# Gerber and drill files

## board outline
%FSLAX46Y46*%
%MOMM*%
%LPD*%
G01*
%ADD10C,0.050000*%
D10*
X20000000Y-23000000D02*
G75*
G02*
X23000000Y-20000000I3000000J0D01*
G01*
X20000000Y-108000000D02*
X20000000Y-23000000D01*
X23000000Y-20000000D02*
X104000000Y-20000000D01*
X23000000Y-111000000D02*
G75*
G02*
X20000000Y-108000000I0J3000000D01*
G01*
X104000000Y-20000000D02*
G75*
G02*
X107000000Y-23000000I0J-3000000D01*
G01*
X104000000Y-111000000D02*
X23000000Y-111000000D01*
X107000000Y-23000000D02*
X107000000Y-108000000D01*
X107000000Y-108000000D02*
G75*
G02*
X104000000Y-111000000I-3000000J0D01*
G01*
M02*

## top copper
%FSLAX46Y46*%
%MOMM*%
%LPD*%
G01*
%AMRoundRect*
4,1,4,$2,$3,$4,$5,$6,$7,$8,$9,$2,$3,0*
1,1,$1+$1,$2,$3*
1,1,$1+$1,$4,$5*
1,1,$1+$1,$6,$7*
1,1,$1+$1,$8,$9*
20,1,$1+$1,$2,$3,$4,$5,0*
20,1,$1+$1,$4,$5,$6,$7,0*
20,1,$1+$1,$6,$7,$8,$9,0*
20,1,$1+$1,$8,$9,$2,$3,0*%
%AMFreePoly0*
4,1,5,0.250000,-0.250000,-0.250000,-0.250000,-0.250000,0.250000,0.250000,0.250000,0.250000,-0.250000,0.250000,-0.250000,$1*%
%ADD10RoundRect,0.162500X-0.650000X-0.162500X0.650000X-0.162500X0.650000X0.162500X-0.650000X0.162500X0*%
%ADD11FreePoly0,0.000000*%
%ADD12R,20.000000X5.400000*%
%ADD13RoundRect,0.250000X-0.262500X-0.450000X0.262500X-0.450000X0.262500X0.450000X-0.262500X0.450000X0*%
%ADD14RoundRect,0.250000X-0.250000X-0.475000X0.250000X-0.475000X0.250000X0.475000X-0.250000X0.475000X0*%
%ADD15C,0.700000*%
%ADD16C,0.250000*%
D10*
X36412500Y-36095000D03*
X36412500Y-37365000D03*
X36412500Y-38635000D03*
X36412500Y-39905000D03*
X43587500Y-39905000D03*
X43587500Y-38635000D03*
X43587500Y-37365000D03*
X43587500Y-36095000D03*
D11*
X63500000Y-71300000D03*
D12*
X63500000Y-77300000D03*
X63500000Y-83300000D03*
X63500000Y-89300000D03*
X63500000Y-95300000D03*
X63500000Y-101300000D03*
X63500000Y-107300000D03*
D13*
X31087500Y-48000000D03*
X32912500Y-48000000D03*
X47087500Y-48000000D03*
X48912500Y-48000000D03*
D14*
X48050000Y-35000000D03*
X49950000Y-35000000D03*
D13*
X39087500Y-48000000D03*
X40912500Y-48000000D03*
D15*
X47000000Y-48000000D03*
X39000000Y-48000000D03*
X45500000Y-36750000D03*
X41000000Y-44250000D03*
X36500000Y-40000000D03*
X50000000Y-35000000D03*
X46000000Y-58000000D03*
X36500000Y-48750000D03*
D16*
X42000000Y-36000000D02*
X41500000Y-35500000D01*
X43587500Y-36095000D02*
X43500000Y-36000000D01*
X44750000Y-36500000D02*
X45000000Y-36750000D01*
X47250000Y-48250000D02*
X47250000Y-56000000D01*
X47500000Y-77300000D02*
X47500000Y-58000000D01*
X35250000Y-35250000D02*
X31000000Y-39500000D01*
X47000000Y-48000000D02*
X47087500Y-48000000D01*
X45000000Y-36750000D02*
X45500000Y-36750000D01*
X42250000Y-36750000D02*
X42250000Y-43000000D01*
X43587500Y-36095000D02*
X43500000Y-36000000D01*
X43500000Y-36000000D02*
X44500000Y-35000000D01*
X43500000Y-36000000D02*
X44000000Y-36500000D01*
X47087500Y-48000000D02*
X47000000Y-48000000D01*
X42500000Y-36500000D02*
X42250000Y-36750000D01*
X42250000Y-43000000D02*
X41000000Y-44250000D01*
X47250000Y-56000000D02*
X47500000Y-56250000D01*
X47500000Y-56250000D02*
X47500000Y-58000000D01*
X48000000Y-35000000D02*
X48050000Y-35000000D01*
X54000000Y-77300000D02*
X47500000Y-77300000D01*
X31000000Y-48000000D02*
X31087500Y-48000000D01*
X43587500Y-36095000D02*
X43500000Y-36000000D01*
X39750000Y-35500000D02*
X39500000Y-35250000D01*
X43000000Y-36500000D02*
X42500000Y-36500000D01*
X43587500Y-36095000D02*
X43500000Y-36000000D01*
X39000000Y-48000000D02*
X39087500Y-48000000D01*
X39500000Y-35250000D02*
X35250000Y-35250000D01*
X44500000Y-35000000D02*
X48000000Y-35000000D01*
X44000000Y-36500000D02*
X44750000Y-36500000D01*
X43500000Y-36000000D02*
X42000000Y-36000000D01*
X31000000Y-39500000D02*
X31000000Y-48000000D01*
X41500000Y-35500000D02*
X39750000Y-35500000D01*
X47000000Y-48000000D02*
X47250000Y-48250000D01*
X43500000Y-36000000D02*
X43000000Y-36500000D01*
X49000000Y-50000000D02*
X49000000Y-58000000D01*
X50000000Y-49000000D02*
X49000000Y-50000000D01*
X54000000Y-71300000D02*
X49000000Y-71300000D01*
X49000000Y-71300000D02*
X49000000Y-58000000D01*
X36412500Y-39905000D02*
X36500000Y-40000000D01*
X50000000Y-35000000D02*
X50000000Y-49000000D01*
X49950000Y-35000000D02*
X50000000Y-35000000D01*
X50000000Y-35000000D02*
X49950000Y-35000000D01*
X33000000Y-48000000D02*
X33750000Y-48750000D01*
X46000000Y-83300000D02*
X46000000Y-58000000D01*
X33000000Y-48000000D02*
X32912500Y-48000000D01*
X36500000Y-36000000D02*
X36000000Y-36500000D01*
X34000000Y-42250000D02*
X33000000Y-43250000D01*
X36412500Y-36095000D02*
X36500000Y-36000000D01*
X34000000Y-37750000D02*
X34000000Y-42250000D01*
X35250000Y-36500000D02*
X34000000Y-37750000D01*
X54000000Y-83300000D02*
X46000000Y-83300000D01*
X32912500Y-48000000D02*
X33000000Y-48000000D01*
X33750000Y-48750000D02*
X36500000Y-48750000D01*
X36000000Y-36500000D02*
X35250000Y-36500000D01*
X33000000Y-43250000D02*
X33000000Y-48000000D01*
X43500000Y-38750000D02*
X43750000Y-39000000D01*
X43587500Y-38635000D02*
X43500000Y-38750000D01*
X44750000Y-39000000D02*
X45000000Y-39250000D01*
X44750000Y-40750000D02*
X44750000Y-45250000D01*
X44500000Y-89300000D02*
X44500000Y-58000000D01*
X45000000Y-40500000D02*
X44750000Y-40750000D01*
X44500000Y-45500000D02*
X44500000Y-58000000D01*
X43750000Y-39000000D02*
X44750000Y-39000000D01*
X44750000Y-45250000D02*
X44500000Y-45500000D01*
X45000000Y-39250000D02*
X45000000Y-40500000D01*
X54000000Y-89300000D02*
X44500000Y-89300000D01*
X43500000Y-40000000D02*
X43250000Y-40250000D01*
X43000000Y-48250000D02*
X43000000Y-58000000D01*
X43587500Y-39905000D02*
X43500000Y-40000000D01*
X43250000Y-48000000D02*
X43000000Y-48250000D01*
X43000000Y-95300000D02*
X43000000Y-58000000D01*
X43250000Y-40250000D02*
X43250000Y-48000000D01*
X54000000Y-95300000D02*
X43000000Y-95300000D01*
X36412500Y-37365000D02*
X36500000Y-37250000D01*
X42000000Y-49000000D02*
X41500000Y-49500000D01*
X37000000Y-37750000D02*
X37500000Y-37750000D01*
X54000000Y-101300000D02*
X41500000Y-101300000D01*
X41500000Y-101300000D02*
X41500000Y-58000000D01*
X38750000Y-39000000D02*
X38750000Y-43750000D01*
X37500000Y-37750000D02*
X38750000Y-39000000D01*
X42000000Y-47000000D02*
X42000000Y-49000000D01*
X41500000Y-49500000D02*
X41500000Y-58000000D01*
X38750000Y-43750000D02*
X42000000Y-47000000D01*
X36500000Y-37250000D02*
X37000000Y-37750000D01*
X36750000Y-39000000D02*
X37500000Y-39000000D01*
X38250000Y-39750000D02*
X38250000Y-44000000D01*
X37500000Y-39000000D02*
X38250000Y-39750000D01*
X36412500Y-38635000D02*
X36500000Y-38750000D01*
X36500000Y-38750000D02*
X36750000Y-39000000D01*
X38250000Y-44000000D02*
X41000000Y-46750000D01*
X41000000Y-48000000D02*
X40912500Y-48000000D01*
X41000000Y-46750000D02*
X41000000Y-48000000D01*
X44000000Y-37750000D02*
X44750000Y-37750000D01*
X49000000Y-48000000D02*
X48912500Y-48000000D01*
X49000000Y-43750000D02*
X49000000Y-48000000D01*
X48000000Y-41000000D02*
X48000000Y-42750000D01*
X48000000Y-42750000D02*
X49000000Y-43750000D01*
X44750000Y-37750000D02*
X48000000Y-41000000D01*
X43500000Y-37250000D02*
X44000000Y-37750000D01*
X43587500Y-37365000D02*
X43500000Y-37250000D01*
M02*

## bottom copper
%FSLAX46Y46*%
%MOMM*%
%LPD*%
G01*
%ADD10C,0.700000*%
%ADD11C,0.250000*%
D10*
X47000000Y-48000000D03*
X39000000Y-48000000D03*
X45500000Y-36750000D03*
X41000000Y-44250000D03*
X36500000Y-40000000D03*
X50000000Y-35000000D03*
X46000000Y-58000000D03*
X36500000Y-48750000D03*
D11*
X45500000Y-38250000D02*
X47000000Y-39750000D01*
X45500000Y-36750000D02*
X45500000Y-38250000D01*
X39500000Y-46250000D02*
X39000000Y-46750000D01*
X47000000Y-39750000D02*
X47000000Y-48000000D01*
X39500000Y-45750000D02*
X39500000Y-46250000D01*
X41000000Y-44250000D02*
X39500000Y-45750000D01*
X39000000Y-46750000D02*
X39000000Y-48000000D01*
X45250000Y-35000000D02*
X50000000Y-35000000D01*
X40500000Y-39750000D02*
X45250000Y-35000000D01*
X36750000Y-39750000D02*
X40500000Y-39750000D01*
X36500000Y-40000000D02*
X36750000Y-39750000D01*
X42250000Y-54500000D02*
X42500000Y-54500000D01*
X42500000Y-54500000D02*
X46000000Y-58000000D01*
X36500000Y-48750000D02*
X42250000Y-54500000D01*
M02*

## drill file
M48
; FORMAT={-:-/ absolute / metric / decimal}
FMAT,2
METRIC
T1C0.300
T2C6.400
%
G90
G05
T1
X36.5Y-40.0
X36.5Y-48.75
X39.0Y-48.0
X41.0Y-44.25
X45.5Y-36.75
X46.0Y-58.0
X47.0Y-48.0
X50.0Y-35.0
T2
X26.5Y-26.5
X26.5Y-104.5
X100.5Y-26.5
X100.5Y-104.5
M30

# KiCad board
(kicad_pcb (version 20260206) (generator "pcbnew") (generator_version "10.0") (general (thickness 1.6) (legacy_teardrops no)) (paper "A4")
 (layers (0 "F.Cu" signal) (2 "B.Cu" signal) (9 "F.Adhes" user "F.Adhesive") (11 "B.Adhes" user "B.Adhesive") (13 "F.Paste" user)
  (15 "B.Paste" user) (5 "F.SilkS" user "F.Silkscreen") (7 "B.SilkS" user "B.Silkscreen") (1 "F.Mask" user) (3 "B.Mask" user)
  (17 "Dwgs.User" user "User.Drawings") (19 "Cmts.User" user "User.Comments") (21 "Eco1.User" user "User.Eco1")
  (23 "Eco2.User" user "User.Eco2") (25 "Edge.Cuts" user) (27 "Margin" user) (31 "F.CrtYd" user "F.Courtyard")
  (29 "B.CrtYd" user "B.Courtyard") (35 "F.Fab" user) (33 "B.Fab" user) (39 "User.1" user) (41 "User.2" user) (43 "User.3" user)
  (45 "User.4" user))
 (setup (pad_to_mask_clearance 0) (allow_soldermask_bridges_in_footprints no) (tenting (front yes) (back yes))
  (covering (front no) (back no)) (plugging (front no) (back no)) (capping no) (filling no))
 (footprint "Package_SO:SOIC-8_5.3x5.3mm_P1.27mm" (layer "F.Cu") (at 40 38)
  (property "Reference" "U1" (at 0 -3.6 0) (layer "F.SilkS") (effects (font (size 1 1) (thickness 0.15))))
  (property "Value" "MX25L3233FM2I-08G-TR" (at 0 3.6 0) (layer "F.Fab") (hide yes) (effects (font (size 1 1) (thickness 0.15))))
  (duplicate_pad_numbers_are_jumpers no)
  (pad "1" smd roundrect (at -3.5875 -1.905) (size 1.625 0.65) (layers "F.Cu" "F.Mask" "F.Paste") (roundrect_rratio 0.25) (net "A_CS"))
  (pad "2" smd roundrect (at -3.5875 -0.635) (size 1.625 0.65) (layers "F.Cu" "F.Mask" "F.Paste") (roundrect_rratio 0.25) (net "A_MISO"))
  (pad "3" smd roundrect (at -3.5875 0.635) (size 1.625 0.65) (layers "F.Cu" "F.Mask" "F.Paste") (roundrect_rratio 0.25) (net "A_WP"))
  (pad "4" smd roundrect (at -3.5875 1.905) (size 1.625 0.65) (layers "F.Cu" "F.Mask" "F.Paste") (roundrect_rratio 0.25) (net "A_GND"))
  (pad "5" smd roundrect (at 3.5875 1.905) (size 1.625 0.65) (layers "F.Cu" "F.Mask" "F.Paste") (roundrect_rratio 0.25) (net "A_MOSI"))
  (pad "6" smd roundrect (at 3.5875 0.635) (size 1.625 0.65) (layers "F.Cu" "F.Mask" "F.Paste") (roundrect_rratio 0.25) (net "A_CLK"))
  (pad "7" smd roundrect (at 3.5875 -0.635) (size 1.625 0.65) (layers "F.Cu" "F.Mask" "F.Paste") (roundrect_rratio 0.25) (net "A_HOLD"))
  (pad "8" smd roundrect (at 3.5875 -1.905) (size 1.625 0.65) (layers "F.Cu" "F.Mask" "F.Paste") (roundrect_rratio 0.25) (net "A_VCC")))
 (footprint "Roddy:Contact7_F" (layer "F.Cu") (at 63.5 0)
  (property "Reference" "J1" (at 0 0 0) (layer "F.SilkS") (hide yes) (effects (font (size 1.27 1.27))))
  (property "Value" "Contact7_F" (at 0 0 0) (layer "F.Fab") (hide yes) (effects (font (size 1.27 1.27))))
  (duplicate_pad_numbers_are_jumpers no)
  (pad "1" smd custom (at 0 71.3) (size 0.5 0.5) (layers "F.Cu" "F.Mask") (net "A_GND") (solder_mask_margin 0.05) (thermal_bridge_angle 45)
   (options (clearance outline) (anchor rect)) (primitives))
  (pad "2" smd rect (at 0 77.3) (size 20 5.4) (layers "F.Cu" "F.Mask") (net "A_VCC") (solder_mask_margin 0.05) (thermal_bridge_angle 45))
  (pad "3" smd rect (at 0 83.3) (size 20 5.4) (layers "F.Cu" "F.Mask") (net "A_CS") (solder_mask_margin 0.05) (thermal_bridge_angle 45))
  (pad "4" smd rect (at 0 89.3) (size 20 5.4) (layers "F.Cu" "F.Mask") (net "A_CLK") (solder_mask_margin 0.05) (thermal_bridge_angle 45))
  (pad "5" smd rect (at 0 95.3) (size 20 5.4) (layers "F.Cu" "F.Mask") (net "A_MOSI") (solder_mask_margin 0.05) (thermal_bridge_angle 45))
  (pad "6" smd rect (at 0 101.3) (size 20 5.4) (layers "F.Cu" "F.Mask") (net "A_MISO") (solder_mask_margin 0.05) (thermal_bridge_angle 45))
  (pad "7" smd rect (at 0 107.3) (size 20 5.4) (layers "F.Cu" "F.Mask") (solder_mask_margin 0.05) (thermal_bridge_angle 45)))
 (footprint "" (layer "F.Cu") (at 100.5 26.5)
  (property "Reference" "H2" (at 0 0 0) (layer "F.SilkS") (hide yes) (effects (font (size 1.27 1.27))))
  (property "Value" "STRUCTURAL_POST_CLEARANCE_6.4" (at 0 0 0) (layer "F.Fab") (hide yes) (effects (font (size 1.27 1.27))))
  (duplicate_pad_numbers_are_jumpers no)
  (pad "" np_thru_hole circle (at 0 0) (size 6.4 6.4) (drill 6.4) (layers "*.Cu")))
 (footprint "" (layer "F.Cu") (at 26.5 26.5)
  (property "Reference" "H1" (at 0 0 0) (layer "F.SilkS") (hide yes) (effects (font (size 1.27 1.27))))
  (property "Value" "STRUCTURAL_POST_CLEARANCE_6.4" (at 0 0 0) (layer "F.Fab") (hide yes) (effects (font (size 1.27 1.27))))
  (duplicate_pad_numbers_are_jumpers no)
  (pad "" np_thru_hole circle (at 0 0) (size 6.4 6.4) (drill 6.4) (layers "*.Cu")))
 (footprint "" (layer "F.Cu") (at 26.5 104.5)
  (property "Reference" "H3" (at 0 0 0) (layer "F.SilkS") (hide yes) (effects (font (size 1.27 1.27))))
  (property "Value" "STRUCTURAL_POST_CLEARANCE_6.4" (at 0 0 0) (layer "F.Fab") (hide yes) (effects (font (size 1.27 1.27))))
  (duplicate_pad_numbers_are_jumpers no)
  (pad "" np_thru_hole circle (at 0 0) (size 6.4 6.4) (drill 6.4) (layers "*.Cu")))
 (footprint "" (layer "F.Cu") (at 100.5 104.5)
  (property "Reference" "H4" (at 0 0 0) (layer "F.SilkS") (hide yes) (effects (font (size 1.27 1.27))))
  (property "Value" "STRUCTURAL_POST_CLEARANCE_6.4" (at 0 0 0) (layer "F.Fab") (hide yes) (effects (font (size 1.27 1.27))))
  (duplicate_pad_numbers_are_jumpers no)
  (pad "" np_thru_hole circle (at 0 0) (size 6.4 6.4) (drill 6.4) (layers "*.Cu")))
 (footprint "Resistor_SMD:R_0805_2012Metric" (layer "F.Cu") (at 32 48)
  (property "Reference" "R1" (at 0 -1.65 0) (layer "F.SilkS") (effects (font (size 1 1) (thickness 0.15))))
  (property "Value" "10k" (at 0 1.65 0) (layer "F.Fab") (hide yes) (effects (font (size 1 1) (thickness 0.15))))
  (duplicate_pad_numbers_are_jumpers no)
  (pad "1" smd roundrect (at -0.9125 0) (size 1.025 1.4) (layers "F.Cu" "F.Mask" "F.Paste") (roundrect_rratio 0.243902) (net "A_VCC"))
  (pad "2" smd roundrect (at 0.9125 0) (size 1.025 1.4) (layers "F.Cu" "F.Mask" "F.Paste") (roundrect_rratio 0.243902) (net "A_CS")))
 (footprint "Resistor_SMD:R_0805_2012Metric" (layer "F.Cu") (at 48 48)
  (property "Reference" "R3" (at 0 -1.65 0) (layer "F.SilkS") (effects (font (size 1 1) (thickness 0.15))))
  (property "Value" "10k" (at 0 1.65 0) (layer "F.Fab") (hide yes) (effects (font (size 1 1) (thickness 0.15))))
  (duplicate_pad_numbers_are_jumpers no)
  (pad "1" smd roundrect (at -0.9125 0) (size 1.025 1.4) (layers "F.Cu" "F.Mask" "F.Paste") (roundrect_rratio 0.243902) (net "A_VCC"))
  (pad "2" smd roundrect (at 0.9125 0) (size 1.025 1.4) (layers "F.Cu" "F.Mask" "F.Paste") (roundrect_rratio 0.243902) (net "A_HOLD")))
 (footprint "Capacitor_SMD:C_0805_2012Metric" (layer "F.Cu") (at 49 35)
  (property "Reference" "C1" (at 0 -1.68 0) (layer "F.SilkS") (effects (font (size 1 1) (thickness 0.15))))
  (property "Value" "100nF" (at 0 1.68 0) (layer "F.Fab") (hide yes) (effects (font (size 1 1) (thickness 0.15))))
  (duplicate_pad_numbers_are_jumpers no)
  (pad "1" smd roundrect (at -0.95 0) (size 1 1.45) (layers "F.Cu" "F.Mask" "F.Paste") (roundrect_rratio 0.25) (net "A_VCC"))
  (pad "2" smd roundrect (at 0.95 0) (size 1 1.45) (layers "F.Cu" "F.Mask" "F.Paste") (roundrect_rratio 0.25) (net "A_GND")))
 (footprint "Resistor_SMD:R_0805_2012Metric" (layer "F.Cu") (at 40 48)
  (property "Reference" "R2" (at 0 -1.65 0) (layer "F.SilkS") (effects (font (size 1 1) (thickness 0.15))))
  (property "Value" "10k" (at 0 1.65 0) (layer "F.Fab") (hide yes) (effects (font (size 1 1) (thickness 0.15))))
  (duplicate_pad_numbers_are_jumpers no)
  (pad "1" smd roundrect (at -0.9125 0) (size 1.025 1.4) (layers "F.Cu" "F.Mask" "F.Paste") (roundrect_rratio 0.243902) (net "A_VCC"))
  (pad "2" smd roundrect (at 0.9125 0) (size 1.025 1.4) (layers "F.Cu" "F.Mask" "F.Paste") (roundrect_rratio 0.243902) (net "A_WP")))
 (gr_arc (start 20 23) (mid 20.878679 20.878679) (end 23 20) (stroke (width 0.05) (type default)) (layer "Edge.Cuts"))
 (gr_line (start 20 108) (end 20 23) (stroke (width 0.05) (type default)) (layer "Edge.Cuts"))
 (gr_line (start 23 20) (end 104 20) (stroke (width 0.05) (type default)) (layer "Edge.Cuts"))
 (gr_arc (start 23 111) (mid 20.878679 110.12132) (end 20 108) (stroke (width 0.05) (type default)) (layer "Edge.Cuts"))
 (gr_arc (start 104 20) (mid 106.12132 20.878679) (end 107 23) (stroke (width 0.05) (type default)) (layer "Edge.Cuts"))
 (gr_line (start 104 111) (end 23 111) (stroke (width 0.05) (type default)) (layer "Edge.Cuts"))
 (gr_line (start 107 23) (end 107 108) (stroke (width 0.05) (type default)) (layer "Edge.Cuts"))
 (gr_arc (start 107 108) (mid 106.12132 110.12132) (end 104 111) (stroke (width 0.05) (type default)) (layer "Edge.Cuts"))
 (segment (start 42 36) (end 41.5 35.5) (width 0.25) (layer "F.Cu") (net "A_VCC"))
 (segment (start 43.5875 36.095) (end 43.5 36) (width 0.25) (layer "F.Cu") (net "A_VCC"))
 (segment (start 44.75 36.5) (end 45 36.75) (width 0.25) (layer "F.Cu") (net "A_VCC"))
 (segment (start 47.25 48.25) (end 47.25 56) (width 0.25) (layer "F.Cu") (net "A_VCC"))
 (segment (start 47.5 77.3) (end 47.5 58) (width 0.25) (layer "F.Cu") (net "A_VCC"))
 (segment (start 35.25 35.25) (end 31 39.5) (width 0.25) (layer "F.Cu") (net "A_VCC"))
 (segment (start 47 48) (end 47.0875 48) (width 0.25) (layer "F.Cu") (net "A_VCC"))
 (segment (start 45 36.75) (end 45.5 36.75) (width 0.25) (layer "F.Cu") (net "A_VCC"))
 (segment (start 42.25 36.75) (end 42.25 43) (width 0.25) (layer "F.Cu") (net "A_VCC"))
 (segment (start 43.5875 36.095) (end 43.5 36) (width 0.25) (layer "F.Cu") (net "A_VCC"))
 (segment (start 43.5 36) (end 44.5 35) (width 0.25) (layer "F.Cu") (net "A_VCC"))
 (segment (start 43.5 36) (end 44 36.5) (width 0.25) (layer "F.Cu") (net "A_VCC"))
 (segment (start 47.0875 48) (end 47 48) (width 0.25) (layer "F.Cu") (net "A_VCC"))
 (segment (start 42.5 36.5) (end 42.25 36.75) (width 0.25) (layer "F.Cu") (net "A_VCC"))
 (segment (start 42.25 43) (end 41 44.25) (width 0.25) (layer "F.Cu") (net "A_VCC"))
 (segment (start 47.25 56) (end 47.5 56.25) (width 0.25) (layer "F.Cu") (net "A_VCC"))
 (segment (start 47.5 56.25) (end 47.5 58) (width 0.25) (layer "F.Cu") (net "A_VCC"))
 (segment (start 48 35) (end 48.05 35) (width 0.25) (layer "F.Cu") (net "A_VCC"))
 (segment (start 54 77.3) (end 47.5 77.3) (width 0.25) (layer "F.Cu") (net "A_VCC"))
 (segment (start 31 48) (end 31.0875 48) (width 0.25) (layer "F.Cu") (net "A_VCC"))
 (segment (start 43.5875 36.095) (end 43.5 36) (width 0.25) (layer "F.Cu") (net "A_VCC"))
 (segment (start 39.75 35.5) (end 39.5 35.25) (width 0.25) (layer "F.Cu") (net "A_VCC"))
 (segment (start 43 36.5) (end 42.5 36.5) (width 0.25) (layer "F.Cu") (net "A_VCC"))
 (segment (start 43.5875 36.095) (end 43.5 36) (width 0.25) (layer "F.Cu") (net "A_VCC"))
 (segment (start 39 48) (end 39.0875 48) (width 0.25) (layer "F.Cu") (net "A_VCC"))
 (segment (start 39.5 35.25) (end 35.25 35.25) (width 0.25) (layer "F.Cu") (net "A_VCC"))
 (segment (start 44.5 35) (end 48 35) (width 0.25) (layer "F.Cu") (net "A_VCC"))
 (segment (start 44 36.5) (end 44.75 36.5) (width 0.25) (layer "F.Cu") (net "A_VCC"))
 (segment (start 43.5 36) (end 42 36) (width 0.25) (layer "F.Cu") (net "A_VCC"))
 (segment (start 31 39.5) (end 31 48) (width 0.25) (layer "F.Cu") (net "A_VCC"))
 (segment (start 41.5 35.5) (end 39.75 35.5) (width 0.25) (layer "F.Cu") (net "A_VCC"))
 (segment (start 47 48) (end 47.25 48.25) (width 0.25) (layer "F.Cu") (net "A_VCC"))
 (segment (start 43.5 36) (end 43 36.5) (width 0.25) (layer "F.Cu") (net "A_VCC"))
 (via (at 47 48) (size 0.7) (drill 0.3) (layers "F.Cu" "B.Cu") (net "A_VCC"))
 (via (at 39 48) (size 0.7) (drill 0.3) (layers "F.Cu" "B.Cu") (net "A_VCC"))
 (via (at 45.5 36.75) (size 0.7) (drill 0.3) (layers "F.Cu" "B.Cu") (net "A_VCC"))
 (via (at 41 44.25) (size 0.7) (drill 0.3) (layers "F.Cu" "B.Cu") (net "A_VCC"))
 (segment (start 45.5 38.25) (end 47 39.75) (width 0.25) (layer "B.Cu") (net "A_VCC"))
 (segment (start 45.5 36.75) (end 45.5 38.25) (width 0.25) (layer "B.Cu") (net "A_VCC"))
 (segment (start 39.5 46.25) (end 39 46.75) (width 0.25) (layer "B.Cu") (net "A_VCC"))
 (segment (start 47 39.75) (end 47 48) (width 0.25) (layer "B.Cu") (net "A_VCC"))
 (segment (start 39.5 45.75) (end 39.5 46.25) (width 0.25) (layer "B.Cu") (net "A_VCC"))
 (segment (start 41 44.25) (end 39.5 45.75) (width 0.25) (layer "B.Cu") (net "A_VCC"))
 (segment (start 39 46.75) (end 39 48) (width 0.25) (layer "B.Cu") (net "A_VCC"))
 (segment (start 49 50) (end 49 58) (width 0.25) (layer "F.Cu") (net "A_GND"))
 (segment (start 50 49) (end 49 50) (width 0.25) (layer "F.Cu") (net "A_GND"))
 (segment (start 54 71.3) (end 49 71.3) (width 0.25) (layer "F.Cu") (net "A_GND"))
 (segment (start 49 71.3) (end 49 58) (width 0.25) (layer "F.Cu") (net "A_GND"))
 (segment (start 36.4125 39.905) (end 36.5 40) (width 0.25) (layer "F.Cu") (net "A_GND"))
 (segment (start 50 35) (end 50 49) (width 0.25) (layer "F.Cu") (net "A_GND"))
 (segment (start 49.95 35) (end 50 35) (width 0.25) (layer "F.Cu") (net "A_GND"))
 (segment (start 50 35) (end 49.95 35) (width 0.25) (layer "F.Cu") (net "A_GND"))
 (via (at 36.5 40) (size 0.7) (drill 0.3) (layers "F.Cu" "B.Cu") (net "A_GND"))
 (via (at 50 35) (size 0.7) (drill 0.3) (layers "F.Cu" "B.Cu") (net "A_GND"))
 (segment (start 45.25 35) (end 50 35) (width 0.25) (layer "B.Cu") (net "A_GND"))
 (segment (start 40.5 39.75) (end 45.25 35) (width 0.25) (layer "B.Cu") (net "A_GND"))
 (segment (start 36.75 39.75) (end 40.5 39.75) (width 0.25) (layer "B.Cu") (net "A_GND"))
 (segment (start 36.5 40) (end 36.75 39.75) (width 0.25) (layer "B.Cu") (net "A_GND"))
 (segment (start 33 48) (end 33.75 48.75) (width 0.25) (layer "F.Cu") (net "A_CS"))
 (segment (start 46 83.3) (end 46 58) (width 0.25) (layer "F.Cu") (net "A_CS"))
 (segment (start 33 48) (end 32.9125 48) (width 0.25) (layer "F.Cu") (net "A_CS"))
 (segment (start 36.5 36) (end 36 36.5) (width 0.25) (layer "F.Cu") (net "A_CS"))
 (segment (start 34 42.25) (end 33 43.25) (width 0.25) (layer "F.Cu") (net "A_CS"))
 (segment (start 36.4125 36.095) (end 36.5 36) (width 0.25) (layer "F.Cu") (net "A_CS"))
 (segment (start 34 37.75) (end 34 42.25) (width 0.25) (layer "F.Cu") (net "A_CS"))
 (segment (start 35.25 36.5) (end 34 37.75) (width 0.25) (layer "F.Cu") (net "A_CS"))
 (segment (start 54 83.3) (end 46 83.3) (width 0.25) (layer "F.Cu") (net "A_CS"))
 (segment (start 32.9125 48) (end 33 48) (width 0.25) (layer "F.Cu") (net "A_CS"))
 (segment (start 33.75 48.75) (end 36.5 48.75) (width 0.25) (layer "F.Cu") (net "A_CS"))
 (segment (start 36 36.5) (end 35.25 36.5) (width 0.25) (layer "F.Cu") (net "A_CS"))
 (segment (start 33 43.25) (end 33 48) (width 0.25) (layer "F.Cu") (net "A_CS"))
 (via (at 46 58) (size 0.7) (drill 0.3) (layers "F.Cu" "B.Cu") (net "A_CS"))
 (via (at 36.5 48.75) (size 0.7) (drill 0.3) (layers "F.Cu" "B.Cu") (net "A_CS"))
 (segment (start 42.25 54.5) (end 42.5 54.5) (width 0.25) (layer "B.Cu") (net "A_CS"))
 (segment (start 42.5 54.5) (end 46 58) (width 0.25) (layer "B.Cu") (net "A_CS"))
 (segment (start 36.5 48.75) (end 42.25 54.5) (width 0.25) (layer "B.Cu") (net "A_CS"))
 (segment (start 43.5 38.75) (end 43.75 39) (width 0.25) (layer "F.Cu") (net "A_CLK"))
 (segment (start 43.5875 38.635) (end 43.5 38.75) (width 0.25) (layer "F.Cu") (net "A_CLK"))
 (segment (start 44.75 39) (end 45 39.25) (width 0.25) (layer "F.Cu") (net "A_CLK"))
 (segment (start 44.75 40.75) (end 44.75 45.25) (width 0.25) (layer "F.Cu") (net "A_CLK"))
 (segment (start 44.5 89.3) (end 44.5 58) (width 0.25) (layer "F.Cu") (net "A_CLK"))
 (segment (start 45 40.5) (end 44.75 40.75) (width 0.25) (layer "F.Cu") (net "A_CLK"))
 (segment (start 44.5 45.5) (end 44.5 58) (width 0.25) (layer "F.Cu") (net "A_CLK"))
 (segment (start 43.75 39) (end 44.75 39) (width 0.25) (layer "F.Cu") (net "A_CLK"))
 (segment (start 44.75 45.25) (end 44.5 45.5) (width 0.25) (layer "F.Cu") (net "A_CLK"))
 (segment (start 45 39.25) (end 45 40.5) (width 0.25) (layer "F.Cu") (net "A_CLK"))
 (segment (start 54 89.3) (end 44.5 89.3) (width 0.25) (layer "F.Cu") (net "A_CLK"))
 (segment (start 43.5 40) (end 43.25 40.25) (width 0.25) (layer "F.Cu") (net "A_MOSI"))
 (segment (start 43 48.25) (end 43 58) (width 0.25) (layer "F.Cu") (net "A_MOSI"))
 (segment (start 43.5875 39.905) (end 43.5 40) (width 0.25) (layer "F.Cu") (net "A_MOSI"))
 (segment (start 43.25 48) (end 43 48.25) (width 0.25) (layer "F.Cu") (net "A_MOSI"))
 (segment (start 43 95.3) (end 43 58) (width 0.25) (layer "F.Cu") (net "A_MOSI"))
 (segment (start 43.25 40.25) (end 43.25 48) (width 0.25) (layer "F.Cu") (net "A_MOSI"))
 (segment (start 54 95.3) (end 43 95.3) (width 0.25) (layer "F.Cu") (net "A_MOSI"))
 (segment (start 36.4125 37.365) (end 36.5 37.25) (width 0.25) (layer "F.Cu") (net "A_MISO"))
 (segment (start 42 49) (end 41.5 49.5) (width 0.25) (layer "F.Cu") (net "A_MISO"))
 (segment (start 37 37.75) (end 37.5 37.75) (width 0.25) (layer "F.Cu") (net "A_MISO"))
 (segment (start 54 101.3) (end 41.5 101.3) (width 0.25) (layer "F.Cu") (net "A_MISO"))
 (segment (start 41.5 101.3) (end 41.5 58) (width 0.25) (layer "F.Cu") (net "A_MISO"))
 (segment (start 38.75 39) (end 38.75 43.75) (width 0.25) (layer "F.Cu") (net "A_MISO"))
 (segment (start 37.5 37.75) (end 38.75 39) (width 0.25) (layer "F.Cu") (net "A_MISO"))
 (segment (start 42 47) (end 42 49) (width 0.25) (layer "F.Cu") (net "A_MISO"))
 (segment (start 41.5 49.5) (end 41.5 58) (width 0.25) (layer "F.Cu") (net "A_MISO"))
 (segment (start 38.75 43.75) (end 42 47) (width 0.25) (layer "F.Cu") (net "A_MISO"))
 (segment (start 36.5 37.25) (end 37 37.75) (width 0.25) (layer "F.Cu") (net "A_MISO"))
 (segment (start 36.75 39) (end 37.5 39) (width 0.25) (layer "F.Cu") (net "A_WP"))
 (segment (start 38.25 39.75) (end 38.25 44) (width 0.25) (layer "F.Cu") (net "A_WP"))
 (segment (start 37.5 39) (end 38.25 39.75) (width 0.25) (layer "F.Cu") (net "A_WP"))
 (segment (start 36.4125 38.635) (end 36.5 38.75) (width 0.25) (layer "F.Cu") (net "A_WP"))
 (segment (start 36.5 38.75) (end 36.75 39) (width 0.25) (layer "F.Cu") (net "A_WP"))
 (segment (start 38.25 44) (end 41 46.75) (width 0.25) (layer "F.Cu") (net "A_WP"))
 (segment (start 41 48) (end 40.9125 48) (width 0.25) (layer "F.Cu") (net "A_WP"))
 (segment (start 41 46.75) (end 41 48) (width 0.25) (layer "F.Cu") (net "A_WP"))
 (segment (start 44 37.75) (end 44.75 37.75) (width 0.25) (layer "F.Cu") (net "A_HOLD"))
 (segment (start 49 48) (end 48.9125 48) (width 0.25) (layer "F.Cu") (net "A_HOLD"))
 (segment (start 49 43.75) (end 49 48) (width 0.25) (layer "F.Cu") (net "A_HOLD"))
 (segment (start 48 41) (end 48 42.75) (width 0.25) (layer "F.Cu") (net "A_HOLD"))
 (segment (start 48 42.75) (end 49 43.75) (width 0.25) (layer "F.Cu") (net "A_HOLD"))
 (segment (start 44.75 37.75) (end 48 41) (width 0.25) (layer "F.Cu") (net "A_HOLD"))
 (segment (start 43.5 37.25) (end 44 37.75) (width 0.25) (layer "F.Cu") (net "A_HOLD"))
 (segment (start 43.5875 37.365) (end 43.5 37.25) (width 0.25) (layer "F.Cu") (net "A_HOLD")))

